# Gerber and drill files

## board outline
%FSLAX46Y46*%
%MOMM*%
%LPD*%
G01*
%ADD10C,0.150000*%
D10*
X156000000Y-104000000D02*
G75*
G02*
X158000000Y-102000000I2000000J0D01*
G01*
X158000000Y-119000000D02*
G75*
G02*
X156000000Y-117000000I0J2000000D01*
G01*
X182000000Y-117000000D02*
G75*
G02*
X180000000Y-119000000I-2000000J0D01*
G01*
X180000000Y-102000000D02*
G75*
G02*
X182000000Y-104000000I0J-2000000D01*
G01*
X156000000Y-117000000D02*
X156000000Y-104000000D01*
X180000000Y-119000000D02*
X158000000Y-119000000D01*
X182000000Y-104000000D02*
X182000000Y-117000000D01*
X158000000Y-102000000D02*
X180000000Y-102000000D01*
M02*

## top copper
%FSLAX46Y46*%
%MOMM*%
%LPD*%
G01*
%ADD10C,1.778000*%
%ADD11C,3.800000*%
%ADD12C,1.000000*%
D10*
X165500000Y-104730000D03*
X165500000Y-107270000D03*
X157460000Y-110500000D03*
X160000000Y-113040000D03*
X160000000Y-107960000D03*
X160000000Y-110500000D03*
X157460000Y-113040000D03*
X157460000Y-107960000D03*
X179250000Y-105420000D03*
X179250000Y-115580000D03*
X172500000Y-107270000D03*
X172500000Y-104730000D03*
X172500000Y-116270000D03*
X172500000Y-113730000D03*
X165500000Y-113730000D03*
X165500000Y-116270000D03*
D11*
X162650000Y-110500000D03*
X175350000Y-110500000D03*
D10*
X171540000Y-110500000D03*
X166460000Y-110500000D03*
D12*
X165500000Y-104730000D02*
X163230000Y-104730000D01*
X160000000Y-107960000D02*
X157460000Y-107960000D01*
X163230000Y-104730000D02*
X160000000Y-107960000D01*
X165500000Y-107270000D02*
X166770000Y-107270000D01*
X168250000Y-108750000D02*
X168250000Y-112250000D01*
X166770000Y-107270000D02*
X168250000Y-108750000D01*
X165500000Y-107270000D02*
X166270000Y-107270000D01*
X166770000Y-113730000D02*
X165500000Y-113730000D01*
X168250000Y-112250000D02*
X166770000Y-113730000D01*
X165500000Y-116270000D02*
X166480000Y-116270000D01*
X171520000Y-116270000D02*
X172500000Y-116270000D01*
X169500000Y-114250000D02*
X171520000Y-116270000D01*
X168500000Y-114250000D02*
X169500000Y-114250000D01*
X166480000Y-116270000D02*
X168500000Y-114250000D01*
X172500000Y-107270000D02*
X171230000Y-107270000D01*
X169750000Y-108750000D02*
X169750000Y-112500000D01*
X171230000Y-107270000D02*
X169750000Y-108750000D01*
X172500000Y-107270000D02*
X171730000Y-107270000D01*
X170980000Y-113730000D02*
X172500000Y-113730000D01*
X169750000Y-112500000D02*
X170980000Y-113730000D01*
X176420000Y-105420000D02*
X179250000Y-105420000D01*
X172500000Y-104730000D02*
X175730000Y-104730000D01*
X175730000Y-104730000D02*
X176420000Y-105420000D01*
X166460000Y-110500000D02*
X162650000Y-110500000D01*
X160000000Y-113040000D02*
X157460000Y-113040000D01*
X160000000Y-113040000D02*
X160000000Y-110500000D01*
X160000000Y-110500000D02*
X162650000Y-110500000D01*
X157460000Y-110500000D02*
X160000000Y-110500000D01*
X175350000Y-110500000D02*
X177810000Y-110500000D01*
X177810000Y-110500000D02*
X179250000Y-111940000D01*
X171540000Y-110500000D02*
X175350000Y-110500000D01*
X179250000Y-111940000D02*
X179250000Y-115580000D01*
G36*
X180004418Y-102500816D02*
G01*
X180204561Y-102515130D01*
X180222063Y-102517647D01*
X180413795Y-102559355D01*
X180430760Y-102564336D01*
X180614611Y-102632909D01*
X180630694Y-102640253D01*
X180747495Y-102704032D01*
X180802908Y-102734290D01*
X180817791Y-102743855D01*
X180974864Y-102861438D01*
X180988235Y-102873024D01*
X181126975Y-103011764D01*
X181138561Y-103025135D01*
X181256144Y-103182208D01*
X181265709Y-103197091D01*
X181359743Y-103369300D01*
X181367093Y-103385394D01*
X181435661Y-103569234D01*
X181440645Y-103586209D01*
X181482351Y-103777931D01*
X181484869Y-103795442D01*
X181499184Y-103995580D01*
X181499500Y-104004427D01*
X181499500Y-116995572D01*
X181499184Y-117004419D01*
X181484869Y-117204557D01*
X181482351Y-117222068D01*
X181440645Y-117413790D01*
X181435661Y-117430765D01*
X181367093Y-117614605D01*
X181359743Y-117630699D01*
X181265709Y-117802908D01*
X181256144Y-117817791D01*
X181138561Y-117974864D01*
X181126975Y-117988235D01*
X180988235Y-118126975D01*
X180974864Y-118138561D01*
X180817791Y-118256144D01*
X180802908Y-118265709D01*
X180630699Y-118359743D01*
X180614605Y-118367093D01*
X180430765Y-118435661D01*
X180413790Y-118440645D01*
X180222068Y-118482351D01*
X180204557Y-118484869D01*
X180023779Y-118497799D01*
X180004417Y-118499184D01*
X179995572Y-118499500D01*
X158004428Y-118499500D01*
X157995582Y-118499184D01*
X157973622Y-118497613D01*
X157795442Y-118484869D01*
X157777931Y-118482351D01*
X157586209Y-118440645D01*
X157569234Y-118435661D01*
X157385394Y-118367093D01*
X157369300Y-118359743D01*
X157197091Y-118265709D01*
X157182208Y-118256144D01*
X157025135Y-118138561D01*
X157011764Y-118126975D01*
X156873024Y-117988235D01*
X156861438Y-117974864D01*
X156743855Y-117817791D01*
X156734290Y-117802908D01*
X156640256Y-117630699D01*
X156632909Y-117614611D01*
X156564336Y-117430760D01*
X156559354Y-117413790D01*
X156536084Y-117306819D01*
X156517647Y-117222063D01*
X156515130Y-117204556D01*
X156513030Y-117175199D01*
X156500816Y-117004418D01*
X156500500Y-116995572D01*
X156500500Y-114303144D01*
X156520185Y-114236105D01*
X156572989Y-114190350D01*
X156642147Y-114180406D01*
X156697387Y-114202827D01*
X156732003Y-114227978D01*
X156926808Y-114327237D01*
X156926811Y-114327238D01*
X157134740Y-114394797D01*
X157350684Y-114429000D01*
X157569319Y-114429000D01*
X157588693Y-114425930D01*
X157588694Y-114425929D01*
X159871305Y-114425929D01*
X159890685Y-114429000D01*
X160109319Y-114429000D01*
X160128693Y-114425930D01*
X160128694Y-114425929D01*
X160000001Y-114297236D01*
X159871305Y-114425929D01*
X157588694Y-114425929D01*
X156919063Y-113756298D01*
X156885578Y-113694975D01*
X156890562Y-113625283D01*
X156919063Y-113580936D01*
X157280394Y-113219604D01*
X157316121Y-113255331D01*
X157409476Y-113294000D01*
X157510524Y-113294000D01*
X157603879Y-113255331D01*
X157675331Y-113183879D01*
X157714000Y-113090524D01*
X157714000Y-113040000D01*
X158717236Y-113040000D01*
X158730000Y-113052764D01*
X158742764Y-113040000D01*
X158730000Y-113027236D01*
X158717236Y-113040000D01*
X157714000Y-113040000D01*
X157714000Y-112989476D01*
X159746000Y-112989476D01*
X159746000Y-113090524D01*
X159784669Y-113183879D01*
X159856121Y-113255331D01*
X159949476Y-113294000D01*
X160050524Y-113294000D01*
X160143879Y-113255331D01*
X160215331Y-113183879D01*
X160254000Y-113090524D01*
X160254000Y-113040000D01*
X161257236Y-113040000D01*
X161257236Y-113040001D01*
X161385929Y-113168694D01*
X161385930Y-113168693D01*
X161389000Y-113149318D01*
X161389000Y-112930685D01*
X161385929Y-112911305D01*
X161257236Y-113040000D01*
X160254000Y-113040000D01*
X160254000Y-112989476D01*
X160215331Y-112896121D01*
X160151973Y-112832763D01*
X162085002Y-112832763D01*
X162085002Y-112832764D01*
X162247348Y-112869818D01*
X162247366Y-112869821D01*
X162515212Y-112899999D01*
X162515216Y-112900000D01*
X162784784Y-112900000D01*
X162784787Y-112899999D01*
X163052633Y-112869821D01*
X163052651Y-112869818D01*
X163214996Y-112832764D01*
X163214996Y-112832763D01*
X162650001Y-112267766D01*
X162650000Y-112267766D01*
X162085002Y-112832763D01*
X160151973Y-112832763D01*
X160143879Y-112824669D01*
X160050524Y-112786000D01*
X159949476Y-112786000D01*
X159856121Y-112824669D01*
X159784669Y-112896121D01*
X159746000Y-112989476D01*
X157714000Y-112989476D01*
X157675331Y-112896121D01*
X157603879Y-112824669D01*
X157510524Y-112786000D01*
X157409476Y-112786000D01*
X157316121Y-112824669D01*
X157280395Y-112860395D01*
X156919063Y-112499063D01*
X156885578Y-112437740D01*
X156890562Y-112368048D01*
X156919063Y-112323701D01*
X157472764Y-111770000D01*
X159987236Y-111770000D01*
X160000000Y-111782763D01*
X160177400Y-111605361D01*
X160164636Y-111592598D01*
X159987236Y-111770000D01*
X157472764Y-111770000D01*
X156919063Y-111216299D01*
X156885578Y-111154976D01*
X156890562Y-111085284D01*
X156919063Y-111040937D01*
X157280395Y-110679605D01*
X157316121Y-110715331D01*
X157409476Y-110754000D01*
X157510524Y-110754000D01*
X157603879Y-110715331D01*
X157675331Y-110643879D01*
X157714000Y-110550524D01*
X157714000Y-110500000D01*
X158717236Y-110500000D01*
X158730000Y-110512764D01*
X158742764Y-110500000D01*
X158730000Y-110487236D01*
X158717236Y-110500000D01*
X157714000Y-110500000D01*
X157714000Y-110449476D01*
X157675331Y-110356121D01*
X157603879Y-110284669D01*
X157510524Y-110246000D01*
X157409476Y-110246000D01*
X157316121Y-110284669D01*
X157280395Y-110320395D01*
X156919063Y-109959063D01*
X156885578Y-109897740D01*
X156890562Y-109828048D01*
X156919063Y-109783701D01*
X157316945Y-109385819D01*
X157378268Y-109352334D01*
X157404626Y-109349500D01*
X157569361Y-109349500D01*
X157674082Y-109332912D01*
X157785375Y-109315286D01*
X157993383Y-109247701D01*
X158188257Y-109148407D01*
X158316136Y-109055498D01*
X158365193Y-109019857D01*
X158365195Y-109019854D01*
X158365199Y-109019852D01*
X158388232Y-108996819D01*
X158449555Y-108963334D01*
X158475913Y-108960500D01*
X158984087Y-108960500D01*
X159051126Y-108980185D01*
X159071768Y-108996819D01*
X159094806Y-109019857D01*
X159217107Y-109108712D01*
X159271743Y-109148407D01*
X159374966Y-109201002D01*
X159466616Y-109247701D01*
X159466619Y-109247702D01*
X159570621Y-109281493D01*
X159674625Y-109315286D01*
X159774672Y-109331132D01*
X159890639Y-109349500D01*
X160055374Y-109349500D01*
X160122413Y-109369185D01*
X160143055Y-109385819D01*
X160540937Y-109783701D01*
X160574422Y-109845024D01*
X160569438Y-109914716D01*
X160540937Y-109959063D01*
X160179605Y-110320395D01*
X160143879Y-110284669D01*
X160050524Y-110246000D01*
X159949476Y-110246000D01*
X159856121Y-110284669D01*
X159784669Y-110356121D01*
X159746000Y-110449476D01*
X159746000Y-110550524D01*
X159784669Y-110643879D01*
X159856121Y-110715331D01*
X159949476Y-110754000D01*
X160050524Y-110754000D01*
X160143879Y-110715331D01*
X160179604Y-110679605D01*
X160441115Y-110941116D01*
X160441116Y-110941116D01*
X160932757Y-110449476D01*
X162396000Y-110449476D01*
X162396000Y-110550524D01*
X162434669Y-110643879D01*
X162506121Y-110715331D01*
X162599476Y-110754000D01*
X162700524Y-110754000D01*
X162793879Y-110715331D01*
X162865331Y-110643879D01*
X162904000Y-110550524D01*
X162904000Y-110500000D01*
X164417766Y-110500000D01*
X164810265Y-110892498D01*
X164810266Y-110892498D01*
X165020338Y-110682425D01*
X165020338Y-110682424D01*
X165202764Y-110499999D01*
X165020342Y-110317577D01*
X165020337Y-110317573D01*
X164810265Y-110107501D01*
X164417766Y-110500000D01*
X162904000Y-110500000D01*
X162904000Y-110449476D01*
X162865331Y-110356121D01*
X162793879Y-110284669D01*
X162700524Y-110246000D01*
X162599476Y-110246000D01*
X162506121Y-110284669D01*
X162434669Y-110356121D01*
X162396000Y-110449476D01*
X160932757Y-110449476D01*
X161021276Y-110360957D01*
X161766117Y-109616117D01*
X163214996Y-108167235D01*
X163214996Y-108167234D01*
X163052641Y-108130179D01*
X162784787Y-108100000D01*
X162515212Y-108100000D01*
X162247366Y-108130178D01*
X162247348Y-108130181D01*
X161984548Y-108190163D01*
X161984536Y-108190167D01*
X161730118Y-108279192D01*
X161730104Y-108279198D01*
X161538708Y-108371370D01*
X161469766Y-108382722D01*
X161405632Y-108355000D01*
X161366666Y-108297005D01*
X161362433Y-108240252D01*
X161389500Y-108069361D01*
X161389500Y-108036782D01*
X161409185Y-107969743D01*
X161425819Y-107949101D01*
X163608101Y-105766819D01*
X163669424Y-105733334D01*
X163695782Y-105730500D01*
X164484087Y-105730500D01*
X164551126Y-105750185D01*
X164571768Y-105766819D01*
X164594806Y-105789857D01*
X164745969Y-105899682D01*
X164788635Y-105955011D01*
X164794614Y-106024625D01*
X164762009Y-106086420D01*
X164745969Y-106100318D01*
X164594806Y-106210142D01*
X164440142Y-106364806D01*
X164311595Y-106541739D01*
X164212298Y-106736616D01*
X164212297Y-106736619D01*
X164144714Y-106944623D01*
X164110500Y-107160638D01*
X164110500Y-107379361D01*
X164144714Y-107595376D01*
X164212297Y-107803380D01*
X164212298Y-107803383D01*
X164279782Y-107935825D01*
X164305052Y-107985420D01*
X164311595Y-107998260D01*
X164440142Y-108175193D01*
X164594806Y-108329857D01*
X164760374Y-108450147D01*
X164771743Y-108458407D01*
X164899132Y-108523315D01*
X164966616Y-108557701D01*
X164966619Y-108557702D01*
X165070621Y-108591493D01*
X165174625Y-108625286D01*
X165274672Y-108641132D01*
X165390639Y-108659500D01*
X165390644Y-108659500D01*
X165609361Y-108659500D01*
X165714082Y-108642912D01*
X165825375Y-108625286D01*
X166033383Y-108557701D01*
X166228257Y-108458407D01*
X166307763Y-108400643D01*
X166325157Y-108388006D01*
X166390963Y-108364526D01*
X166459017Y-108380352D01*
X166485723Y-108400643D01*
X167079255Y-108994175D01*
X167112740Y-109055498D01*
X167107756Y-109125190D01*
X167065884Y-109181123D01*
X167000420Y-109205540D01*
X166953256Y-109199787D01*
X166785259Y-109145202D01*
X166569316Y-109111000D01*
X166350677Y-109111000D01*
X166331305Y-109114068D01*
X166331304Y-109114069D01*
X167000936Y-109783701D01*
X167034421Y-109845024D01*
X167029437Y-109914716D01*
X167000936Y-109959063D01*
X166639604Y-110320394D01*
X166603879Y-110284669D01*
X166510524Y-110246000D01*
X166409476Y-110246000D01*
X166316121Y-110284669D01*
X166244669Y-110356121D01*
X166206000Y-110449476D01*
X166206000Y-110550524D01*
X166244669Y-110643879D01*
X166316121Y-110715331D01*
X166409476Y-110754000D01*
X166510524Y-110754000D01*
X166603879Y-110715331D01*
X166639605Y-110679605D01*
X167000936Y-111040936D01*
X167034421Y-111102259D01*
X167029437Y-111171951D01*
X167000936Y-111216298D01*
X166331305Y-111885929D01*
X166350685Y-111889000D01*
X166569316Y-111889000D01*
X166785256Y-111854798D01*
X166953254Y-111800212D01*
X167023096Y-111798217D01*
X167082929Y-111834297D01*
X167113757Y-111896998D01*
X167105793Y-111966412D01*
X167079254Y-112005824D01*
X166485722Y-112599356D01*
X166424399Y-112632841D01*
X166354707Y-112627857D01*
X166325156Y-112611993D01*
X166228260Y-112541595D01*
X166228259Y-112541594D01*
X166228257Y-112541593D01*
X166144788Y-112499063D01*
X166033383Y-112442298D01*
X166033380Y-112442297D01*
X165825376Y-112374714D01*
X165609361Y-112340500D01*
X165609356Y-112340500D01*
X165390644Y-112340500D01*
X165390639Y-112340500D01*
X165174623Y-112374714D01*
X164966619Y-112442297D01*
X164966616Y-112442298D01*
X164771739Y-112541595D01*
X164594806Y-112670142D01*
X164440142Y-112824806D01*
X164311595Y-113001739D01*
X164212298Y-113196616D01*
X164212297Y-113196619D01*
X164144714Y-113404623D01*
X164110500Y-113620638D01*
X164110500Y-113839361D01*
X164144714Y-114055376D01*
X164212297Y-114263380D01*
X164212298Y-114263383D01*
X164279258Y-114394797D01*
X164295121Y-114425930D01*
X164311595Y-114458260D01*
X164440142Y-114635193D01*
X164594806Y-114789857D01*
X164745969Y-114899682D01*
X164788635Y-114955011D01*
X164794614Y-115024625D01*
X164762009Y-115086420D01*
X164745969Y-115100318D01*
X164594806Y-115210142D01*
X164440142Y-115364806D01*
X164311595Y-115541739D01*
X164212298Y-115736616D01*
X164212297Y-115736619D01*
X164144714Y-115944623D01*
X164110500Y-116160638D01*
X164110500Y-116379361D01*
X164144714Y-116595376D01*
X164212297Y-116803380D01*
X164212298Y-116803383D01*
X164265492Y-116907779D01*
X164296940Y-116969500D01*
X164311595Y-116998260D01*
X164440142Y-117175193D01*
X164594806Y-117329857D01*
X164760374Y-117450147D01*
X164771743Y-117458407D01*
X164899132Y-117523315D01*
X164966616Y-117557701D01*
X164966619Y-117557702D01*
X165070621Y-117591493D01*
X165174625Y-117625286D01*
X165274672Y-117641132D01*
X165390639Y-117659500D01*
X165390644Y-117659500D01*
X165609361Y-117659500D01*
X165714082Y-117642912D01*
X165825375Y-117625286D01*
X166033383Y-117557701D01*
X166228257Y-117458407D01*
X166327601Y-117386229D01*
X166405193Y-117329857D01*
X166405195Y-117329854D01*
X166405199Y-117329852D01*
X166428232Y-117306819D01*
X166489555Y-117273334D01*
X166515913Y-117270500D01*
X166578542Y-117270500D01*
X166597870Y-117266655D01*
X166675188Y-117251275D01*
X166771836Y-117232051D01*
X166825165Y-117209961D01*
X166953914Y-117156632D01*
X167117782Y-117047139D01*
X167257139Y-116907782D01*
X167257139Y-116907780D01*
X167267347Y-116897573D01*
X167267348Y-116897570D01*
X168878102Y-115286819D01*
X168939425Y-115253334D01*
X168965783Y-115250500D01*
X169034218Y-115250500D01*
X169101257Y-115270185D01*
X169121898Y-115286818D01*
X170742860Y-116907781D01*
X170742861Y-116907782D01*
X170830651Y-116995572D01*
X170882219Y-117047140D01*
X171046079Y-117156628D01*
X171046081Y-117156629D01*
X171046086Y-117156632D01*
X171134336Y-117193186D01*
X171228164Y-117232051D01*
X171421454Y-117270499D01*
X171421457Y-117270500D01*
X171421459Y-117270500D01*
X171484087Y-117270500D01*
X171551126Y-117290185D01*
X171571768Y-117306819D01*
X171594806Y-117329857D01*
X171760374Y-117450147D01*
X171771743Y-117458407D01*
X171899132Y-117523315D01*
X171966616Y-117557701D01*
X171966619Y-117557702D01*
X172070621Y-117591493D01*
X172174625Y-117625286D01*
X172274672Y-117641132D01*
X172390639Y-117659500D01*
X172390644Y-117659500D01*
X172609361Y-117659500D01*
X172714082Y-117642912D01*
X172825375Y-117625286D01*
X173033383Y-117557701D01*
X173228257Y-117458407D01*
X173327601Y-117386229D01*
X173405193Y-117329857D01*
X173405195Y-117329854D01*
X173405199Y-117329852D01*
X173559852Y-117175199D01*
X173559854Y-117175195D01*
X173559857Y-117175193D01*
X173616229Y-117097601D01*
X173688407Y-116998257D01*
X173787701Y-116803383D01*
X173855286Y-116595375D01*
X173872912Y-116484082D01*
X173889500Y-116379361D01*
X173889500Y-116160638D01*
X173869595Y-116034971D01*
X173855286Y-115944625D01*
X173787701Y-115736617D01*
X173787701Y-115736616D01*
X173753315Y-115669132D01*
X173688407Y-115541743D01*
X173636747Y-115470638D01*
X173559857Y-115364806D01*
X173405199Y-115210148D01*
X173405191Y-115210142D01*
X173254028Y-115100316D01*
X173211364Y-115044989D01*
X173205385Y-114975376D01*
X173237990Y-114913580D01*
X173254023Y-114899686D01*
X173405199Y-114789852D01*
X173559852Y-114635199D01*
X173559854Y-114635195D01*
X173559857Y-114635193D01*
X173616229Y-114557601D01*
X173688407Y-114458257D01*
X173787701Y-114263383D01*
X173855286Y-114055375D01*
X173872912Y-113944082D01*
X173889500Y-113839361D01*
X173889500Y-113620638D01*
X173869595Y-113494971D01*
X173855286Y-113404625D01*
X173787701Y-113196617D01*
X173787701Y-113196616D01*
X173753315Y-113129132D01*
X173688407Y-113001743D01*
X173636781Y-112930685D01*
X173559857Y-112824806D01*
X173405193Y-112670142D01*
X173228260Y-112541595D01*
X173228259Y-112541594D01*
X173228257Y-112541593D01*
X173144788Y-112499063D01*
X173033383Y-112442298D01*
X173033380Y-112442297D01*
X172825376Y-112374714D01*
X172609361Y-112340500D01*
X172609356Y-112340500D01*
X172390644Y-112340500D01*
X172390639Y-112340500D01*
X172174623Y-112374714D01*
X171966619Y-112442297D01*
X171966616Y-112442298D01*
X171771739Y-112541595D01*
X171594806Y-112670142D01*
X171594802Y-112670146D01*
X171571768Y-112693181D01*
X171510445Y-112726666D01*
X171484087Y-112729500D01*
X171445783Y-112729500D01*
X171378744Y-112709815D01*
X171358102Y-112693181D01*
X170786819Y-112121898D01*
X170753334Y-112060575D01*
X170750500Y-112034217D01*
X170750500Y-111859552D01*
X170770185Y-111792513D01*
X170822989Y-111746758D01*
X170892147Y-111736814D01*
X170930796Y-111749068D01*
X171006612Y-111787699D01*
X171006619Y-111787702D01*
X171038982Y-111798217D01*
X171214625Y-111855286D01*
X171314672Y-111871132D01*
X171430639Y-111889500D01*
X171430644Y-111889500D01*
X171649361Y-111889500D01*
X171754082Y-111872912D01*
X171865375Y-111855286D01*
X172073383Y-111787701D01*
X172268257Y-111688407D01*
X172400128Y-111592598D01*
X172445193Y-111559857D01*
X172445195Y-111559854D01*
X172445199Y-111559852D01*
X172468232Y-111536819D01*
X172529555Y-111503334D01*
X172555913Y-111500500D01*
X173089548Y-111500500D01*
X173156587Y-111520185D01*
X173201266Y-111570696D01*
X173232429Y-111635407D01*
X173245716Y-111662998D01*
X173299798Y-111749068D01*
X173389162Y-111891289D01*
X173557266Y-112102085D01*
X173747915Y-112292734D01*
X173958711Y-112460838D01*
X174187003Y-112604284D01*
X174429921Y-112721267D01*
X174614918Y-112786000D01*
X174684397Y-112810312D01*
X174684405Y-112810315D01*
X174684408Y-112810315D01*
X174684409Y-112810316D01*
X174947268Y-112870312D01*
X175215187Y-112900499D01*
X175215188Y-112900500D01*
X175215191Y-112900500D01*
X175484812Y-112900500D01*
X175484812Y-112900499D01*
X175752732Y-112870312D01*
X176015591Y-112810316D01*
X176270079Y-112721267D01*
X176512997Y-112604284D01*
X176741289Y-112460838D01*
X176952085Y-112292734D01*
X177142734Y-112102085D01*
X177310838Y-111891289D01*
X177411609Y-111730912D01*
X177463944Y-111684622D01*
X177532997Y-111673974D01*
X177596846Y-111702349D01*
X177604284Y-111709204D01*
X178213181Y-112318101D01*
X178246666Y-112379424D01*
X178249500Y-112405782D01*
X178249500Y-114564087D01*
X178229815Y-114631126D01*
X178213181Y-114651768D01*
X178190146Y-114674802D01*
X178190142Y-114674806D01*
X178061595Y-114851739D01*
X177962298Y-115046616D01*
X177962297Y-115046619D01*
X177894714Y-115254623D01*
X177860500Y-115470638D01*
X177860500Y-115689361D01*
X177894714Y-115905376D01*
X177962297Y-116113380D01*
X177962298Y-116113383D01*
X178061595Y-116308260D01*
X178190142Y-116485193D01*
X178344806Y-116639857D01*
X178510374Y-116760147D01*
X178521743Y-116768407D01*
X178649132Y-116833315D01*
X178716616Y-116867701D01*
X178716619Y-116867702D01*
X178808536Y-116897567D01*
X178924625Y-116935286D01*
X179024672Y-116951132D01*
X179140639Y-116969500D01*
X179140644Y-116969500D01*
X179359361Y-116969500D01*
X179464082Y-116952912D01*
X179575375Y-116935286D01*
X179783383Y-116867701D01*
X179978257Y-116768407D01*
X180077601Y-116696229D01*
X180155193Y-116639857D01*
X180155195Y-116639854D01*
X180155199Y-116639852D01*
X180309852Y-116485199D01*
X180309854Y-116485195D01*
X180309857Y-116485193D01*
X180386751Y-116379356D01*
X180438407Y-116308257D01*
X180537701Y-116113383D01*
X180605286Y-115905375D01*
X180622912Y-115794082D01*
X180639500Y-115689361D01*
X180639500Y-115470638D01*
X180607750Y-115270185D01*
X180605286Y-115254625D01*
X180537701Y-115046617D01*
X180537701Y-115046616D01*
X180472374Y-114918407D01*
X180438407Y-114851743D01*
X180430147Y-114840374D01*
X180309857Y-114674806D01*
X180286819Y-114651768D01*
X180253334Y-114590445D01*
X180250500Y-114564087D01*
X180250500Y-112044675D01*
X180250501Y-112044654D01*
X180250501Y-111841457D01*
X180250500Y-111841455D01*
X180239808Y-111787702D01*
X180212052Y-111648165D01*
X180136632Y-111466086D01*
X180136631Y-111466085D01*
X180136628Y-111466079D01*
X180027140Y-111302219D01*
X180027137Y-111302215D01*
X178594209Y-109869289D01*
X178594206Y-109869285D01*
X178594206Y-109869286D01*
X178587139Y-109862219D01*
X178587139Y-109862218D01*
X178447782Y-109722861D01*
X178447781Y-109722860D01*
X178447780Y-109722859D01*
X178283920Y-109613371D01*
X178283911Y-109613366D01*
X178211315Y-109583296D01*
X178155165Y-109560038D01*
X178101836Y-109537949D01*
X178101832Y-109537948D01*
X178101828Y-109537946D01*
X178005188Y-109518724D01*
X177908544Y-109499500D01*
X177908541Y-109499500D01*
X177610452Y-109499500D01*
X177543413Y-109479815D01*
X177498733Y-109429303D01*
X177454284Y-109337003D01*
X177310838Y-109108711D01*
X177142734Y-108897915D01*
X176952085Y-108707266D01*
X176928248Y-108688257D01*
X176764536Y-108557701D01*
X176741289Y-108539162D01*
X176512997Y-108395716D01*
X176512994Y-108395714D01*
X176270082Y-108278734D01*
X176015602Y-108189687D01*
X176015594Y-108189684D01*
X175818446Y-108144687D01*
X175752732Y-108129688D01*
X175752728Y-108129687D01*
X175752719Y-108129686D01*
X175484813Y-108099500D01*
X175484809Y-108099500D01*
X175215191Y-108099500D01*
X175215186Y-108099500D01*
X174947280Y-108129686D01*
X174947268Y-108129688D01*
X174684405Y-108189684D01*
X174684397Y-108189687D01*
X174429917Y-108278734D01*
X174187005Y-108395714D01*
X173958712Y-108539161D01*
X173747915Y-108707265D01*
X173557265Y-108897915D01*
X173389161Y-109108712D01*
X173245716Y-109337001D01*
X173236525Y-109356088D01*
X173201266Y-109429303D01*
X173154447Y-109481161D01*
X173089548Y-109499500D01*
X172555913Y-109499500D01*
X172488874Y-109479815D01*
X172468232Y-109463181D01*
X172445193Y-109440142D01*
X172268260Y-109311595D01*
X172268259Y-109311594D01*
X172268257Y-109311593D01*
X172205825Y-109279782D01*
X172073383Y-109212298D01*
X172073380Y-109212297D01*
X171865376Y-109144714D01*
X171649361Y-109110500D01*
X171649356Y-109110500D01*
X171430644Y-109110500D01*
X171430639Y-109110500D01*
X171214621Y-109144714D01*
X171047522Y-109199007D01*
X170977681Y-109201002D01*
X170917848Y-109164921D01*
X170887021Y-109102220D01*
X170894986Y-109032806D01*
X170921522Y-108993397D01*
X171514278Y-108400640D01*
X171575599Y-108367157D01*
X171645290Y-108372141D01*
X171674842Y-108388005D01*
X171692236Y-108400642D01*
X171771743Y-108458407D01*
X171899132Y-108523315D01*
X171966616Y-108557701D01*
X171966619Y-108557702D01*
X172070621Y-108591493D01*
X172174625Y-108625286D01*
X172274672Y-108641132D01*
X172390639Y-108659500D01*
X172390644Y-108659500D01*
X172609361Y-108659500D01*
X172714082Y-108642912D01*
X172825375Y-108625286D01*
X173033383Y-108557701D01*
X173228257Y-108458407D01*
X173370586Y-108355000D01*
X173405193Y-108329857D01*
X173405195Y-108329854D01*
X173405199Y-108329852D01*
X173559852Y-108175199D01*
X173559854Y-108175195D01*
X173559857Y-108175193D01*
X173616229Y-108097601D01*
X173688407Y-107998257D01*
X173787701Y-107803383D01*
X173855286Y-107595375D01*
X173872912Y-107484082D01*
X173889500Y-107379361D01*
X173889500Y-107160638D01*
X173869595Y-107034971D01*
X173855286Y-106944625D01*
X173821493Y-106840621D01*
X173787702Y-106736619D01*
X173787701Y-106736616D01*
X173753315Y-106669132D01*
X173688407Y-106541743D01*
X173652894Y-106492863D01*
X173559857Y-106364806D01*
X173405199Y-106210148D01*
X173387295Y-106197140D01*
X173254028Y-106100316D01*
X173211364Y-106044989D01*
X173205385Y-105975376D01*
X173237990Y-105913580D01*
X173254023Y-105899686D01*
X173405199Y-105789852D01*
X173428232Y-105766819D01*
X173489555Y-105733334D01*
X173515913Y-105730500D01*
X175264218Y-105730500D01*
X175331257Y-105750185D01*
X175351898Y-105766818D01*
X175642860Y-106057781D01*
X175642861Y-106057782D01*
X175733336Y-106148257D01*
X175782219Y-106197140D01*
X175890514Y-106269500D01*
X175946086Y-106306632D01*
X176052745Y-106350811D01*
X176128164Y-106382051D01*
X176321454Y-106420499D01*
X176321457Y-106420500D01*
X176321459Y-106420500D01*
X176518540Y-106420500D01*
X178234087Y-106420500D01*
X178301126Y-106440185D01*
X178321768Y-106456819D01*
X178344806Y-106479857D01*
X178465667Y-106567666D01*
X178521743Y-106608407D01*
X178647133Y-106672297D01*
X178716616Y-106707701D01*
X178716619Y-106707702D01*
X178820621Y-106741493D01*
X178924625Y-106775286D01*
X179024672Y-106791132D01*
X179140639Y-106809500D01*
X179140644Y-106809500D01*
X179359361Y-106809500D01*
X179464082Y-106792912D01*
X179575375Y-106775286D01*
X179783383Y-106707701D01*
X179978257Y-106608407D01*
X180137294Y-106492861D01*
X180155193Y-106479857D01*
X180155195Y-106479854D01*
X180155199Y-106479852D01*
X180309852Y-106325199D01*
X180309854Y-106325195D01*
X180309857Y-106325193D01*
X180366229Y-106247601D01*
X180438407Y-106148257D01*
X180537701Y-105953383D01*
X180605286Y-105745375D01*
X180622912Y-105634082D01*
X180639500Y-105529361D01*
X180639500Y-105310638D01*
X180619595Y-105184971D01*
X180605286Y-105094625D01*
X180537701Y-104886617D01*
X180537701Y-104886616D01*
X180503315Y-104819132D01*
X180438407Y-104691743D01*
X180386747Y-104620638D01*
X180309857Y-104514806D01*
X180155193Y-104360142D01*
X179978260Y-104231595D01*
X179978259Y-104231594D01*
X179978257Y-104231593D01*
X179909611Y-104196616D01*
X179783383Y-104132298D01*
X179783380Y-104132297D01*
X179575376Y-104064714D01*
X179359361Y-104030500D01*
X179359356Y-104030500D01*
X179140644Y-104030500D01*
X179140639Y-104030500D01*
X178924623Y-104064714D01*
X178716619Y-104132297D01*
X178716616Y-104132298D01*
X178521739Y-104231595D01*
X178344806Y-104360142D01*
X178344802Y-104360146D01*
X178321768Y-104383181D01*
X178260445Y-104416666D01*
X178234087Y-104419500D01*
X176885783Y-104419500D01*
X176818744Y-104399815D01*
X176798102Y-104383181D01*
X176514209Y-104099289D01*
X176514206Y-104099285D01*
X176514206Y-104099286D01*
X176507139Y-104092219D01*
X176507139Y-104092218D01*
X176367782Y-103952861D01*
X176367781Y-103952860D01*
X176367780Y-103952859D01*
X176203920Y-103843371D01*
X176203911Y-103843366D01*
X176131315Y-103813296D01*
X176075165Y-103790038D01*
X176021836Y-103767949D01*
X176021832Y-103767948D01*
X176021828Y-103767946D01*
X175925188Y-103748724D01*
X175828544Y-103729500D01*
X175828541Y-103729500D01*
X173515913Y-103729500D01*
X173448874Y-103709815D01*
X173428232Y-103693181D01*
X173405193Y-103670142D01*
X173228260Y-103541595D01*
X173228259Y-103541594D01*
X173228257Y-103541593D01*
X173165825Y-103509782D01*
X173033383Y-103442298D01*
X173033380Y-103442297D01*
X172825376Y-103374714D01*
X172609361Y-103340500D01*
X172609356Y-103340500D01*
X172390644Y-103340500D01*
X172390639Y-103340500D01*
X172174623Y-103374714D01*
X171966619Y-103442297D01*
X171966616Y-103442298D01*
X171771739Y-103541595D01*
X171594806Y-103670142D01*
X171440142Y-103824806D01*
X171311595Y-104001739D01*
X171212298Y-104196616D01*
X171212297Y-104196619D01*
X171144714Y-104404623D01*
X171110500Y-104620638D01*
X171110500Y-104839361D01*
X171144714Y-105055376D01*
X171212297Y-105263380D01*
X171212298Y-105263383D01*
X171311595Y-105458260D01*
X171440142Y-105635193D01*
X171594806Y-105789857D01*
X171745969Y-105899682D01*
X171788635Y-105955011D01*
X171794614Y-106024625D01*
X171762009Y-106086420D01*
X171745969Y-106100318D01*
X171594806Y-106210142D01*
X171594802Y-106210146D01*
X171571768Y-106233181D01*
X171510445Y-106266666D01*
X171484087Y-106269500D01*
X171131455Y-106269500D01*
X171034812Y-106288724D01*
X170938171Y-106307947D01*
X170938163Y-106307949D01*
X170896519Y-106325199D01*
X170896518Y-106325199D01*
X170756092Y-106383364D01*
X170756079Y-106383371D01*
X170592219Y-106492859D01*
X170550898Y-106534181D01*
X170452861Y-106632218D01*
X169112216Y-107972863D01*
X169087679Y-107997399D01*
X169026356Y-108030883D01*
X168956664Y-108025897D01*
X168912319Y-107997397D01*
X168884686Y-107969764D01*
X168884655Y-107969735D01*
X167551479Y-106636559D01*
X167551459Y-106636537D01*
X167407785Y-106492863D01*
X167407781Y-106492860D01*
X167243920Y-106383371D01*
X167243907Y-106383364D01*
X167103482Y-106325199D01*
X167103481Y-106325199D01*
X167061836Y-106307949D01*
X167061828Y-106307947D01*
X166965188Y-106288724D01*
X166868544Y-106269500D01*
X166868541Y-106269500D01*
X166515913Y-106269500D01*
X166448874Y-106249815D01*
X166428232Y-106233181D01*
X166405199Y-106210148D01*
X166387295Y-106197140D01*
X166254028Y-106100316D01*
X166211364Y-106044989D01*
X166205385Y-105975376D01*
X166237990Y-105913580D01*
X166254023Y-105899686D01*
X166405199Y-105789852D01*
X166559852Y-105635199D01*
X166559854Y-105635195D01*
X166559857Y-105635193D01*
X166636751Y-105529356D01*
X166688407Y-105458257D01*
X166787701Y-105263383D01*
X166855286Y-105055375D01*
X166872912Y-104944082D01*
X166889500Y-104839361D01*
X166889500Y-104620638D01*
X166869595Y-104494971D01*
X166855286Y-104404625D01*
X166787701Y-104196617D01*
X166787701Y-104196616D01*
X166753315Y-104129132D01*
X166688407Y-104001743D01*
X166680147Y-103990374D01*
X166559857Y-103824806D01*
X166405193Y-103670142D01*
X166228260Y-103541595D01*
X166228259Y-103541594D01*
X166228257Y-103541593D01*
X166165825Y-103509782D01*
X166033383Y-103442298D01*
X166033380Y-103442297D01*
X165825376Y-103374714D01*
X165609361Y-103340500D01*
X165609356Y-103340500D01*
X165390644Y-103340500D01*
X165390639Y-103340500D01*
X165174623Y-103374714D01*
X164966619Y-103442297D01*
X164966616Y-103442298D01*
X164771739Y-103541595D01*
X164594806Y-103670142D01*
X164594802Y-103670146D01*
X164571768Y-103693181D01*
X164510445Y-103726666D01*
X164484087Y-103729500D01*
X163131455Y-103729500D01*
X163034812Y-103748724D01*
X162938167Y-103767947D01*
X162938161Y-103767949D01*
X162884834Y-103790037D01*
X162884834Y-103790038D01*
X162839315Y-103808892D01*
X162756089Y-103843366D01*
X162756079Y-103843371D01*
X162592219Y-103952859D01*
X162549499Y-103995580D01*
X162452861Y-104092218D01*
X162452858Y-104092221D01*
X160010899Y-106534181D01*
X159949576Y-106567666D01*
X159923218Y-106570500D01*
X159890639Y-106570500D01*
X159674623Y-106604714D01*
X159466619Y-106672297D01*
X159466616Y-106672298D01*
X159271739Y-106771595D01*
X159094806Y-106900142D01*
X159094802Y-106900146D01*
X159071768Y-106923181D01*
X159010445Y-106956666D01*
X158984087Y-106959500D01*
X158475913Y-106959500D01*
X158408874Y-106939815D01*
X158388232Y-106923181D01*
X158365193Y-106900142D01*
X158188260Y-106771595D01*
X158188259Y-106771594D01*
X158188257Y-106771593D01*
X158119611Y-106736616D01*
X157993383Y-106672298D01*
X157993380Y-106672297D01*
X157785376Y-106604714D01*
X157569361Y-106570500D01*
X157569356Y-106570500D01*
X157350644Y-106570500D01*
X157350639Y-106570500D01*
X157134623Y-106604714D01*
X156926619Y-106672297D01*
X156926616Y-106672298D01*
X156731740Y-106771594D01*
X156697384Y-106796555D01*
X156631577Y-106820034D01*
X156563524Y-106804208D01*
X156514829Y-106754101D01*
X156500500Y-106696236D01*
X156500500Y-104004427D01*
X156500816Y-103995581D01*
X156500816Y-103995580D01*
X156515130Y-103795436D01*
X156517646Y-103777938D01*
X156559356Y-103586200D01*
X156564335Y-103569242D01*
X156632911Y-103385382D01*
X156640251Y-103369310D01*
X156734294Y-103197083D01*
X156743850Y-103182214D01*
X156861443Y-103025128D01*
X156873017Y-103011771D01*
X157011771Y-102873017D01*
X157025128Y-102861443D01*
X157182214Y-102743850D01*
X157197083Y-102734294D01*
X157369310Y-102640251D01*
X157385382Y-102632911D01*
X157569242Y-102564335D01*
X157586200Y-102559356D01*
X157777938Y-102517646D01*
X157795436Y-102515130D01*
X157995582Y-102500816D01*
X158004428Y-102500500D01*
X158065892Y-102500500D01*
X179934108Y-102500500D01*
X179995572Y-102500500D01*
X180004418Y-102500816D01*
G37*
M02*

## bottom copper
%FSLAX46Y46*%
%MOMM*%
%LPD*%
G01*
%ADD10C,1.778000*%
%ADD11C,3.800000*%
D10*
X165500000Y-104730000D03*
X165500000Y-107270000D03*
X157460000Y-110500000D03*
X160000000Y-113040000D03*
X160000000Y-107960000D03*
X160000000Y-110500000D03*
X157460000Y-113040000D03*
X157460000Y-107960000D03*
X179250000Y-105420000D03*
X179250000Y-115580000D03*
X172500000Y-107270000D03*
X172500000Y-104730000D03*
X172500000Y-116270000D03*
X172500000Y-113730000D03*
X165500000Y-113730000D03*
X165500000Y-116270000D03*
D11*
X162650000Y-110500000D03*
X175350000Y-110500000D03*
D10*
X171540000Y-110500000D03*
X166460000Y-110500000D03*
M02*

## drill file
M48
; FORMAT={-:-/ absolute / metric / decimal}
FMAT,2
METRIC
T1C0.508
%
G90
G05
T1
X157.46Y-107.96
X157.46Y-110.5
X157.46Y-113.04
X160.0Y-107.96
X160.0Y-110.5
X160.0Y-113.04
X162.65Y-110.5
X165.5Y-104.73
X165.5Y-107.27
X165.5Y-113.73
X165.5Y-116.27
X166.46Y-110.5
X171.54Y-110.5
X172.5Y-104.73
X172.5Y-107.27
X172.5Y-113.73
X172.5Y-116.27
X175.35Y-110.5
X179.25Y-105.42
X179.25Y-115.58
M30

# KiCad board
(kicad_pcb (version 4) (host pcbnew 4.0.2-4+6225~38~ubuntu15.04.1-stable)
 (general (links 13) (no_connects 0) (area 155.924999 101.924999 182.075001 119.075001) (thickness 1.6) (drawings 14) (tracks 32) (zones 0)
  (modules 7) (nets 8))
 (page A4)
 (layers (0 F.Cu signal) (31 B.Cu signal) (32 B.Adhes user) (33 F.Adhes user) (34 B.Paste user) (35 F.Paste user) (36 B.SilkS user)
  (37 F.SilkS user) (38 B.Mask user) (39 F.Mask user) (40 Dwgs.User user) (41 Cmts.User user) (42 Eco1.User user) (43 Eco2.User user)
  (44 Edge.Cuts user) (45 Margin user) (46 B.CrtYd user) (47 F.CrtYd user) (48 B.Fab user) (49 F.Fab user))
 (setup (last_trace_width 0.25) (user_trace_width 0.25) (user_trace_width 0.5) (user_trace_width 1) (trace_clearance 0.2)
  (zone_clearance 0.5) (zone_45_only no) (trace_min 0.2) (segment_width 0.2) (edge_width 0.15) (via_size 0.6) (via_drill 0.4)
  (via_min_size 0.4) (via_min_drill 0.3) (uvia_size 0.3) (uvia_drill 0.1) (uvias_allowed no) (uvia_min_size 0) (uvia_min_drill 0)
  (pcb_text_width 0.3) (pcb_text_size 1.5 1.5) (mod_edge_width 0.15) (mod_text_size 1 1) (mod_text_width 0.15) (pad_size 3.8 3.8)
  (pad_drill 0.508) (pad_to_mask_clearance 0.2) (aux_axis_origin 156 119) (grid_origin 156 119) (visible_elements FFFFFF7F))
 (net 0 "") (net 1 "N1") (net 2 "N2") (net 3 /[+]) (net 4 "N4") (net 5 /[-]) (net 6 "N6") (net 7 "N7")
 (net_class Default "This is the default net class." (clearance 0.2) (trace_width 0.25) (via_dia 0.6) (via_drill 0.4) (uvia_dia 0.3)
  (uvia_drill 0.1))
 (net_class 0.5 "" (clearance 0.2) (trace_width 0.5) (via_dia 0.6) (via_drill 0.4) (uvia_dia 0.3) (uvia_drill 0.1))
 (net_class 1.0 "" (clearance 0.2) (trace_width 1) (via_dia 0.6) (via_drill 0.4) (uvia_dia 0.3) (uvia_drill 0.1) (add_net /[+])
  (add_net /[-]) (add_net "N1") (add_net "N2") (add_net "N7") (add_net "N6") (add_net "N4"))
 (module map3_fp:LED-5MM (layer F.Cu) (at 165.5 106 270)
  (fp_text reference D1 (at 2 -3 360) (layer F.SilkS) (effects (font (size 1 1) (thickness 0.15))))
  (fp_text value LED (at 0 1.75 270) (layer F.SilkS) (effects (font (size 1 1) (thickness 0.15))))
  (pad 1 thru_hole circle (at -1.27 0 270) (size 1.778 1.778) (drill 0.508) (layers *.Cu *.Mask F.SilkS) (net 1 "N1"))
  (pad 2 thru_hole circle (at 1.27 0 270) (size 1.778 1.778) (drill 0.508) (layers *.Cu *.Mask F.SilkS) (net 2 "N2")))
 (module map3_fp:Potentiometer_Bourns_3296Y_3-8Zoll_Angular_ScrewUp (layer B.Cu) (at 160 110.5)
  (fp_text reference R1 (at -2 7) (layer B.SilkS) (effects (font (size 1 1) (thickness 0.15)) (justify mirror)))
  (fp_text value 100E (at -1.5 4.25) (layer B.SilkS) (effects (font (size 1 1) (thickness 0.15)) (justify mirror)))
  (pad 3 thru_hole circle (at -2.54 0) (size 1.778 1.778) (drill 0.508) (layers *.Cu *.Mask F.SilkS) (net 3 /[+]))
  (pad 2 thru_hole circle (at 0 2.54) (size 1.778 1.778) (drill 0.508) (layers *.Cu *.Mask F.SilkS) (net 3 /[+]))
  (pad 1 thru_hole circle (at 0 -2.54) (size 1.778 1.778) (drill 0.508) (layers *.Cu *.Mask F.SilkS) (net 1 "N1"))
  (pad 3 thru_hole circle (at 0 0) (size 1.778 1.778) (drill 0.508) (layers *.Cu *.Mask F.SilkS) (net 3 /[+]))
  (pad 2 thru_hole circle (at -2.54 2.54) (size 1.778 1.778) (drill 0.508) (layers *.Cu *.Mask B.SilkS) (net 3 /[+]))
  (pad 1 thru_hole circle (at -2.54 -2.54) (size 1.778 1.778) (drill 0.508) (layers *.Cu *.Mask B.SilkS) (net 1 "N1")))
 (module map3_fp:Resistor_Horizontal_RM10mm (layer B.Cu) (at 179.25 110.5 270)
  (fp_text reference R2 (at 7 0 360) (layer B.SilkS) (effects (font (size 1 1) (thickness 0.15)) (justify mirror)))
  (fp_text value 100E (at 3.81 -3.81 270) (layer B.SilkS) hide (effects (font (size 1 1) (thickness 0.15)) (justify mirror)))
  (pad 1 thru_hole circle (at -5.08 0 270) (size 1.778 1.778) (drill 0.508) (layers *.Cu *.Mask F.SilkS) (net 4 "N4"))
  (pad 2 thru_hole circle (at 5.08 0 270) (size 1.778 1.778) (drill 0.508) (layers *.Cu *.Mask F.SilkS) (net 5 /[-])))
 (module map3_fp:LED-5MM (layer F.Cu) (at 172.5 106 90)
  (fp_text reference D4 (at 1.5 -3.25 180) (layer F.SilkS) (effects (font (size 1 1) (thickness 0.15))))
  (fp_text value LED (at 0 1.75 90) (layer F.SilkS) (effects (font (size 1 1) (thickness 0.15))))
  (pad 1 thru_hole circle (at -1.27 0 90) (size 1.778 1.778) (drill 0.508) (layers *.Cu *.Mask F.SilkS) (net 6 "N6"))
  (pad 2 thru_hole circle (at 1.27 0 90) (size 1.778 1.778) (drill 0.508) (layers *.Cu *.Mask F.SilkS) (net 4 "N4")))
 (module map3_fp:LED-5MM (layer F.Cu) (at 172.5 115 90)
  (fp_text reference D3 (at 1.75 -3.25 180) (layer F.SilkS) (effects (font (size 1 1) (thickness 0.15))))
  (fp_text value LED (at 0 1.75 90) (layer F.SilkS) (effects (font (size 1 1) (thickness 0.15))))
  (pad 1 thru_hole circle (at -1.27 0 90) (size 1.778 1.778) (drill 0.508) (layers *.Cu *.Mask F.SilkS) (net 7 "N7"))
  (pad 2 thru_hole circle (at 1.27 0 90) (size 1.778 1.778) (drill 0.508) (layers *.Cu *.Mask F.SilkS) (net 6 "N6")))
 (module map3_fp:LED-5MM (layer F.Cu) (at 165.5 115 270)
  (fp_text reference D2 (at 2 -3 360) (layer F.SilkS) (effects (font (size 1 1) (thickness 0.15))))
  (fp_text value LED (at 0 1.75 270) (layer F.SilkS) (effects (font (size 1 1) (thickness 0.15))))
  (pad 1 thru_hole circle (at -1.27 0 270) (size 1.778 1.778) (drill 0.508) (layers *.Cu *.Mask F.SilkS) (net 2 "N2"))
  (pad 2 thru_hole circle (at 1.27 0 270) (size 1.778 1.778) (drill 0.508) (layers *.Cu *.Mask F.SilkS) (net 7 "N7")))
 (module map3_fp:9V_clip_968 (layer B.Cu) (at 169 110.5 180)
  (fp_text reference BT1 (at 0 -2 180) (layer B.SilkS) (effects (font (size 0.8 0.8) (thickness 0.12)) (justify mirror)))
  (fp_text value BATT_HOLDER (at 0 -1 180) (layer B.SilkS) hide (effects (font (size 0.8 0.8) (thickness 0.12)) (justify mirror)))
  (pad 1 thru_hole circle (at 6.35 0 180) (size 3.8 3.8) (drill 0.508) (layers *.Cu *.Mask B.SilkS) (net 3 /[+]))
  (pad 2 thru_hole circle (at -6.35 0 180) (size 3.8 3.8) (drill 0.508) (layers *.Cu *.Mask B.SilkS) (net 5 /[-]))
  (pad 2 thru_hole circle (at -2.54 0 180) (size 1.778 1.778) (drill 0.508) (layers *.Cu *.Mask F.SilkS) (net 5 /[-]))
  (pad 1 thru_hole circle (at 2.54 0 180) (size 1.778 1.778) (drill 0.508) (layers *.Cu *.Mask F.SilkS) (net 3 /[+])))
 (gr_arc (start 158 104) (end 156 104) (angle 90) (layer Edge.Cuts) (width 0.15))
 (gr_arc (start 158 117) (end 158 119) (angle 90) (layer Edge.Cuts) (width 0.15))
 (gr_arc (start 180 117) (end 182 117) (angle 90) (layer Edge.Cuts) (width 0.15))
 (gr_arc (start 180 104) (end 180 102) (angle 90) (layer Edge.Cuts) (width 0.15))
 (gr_line (start 156 117) (end 156 104) (angle 90) (layer Edge.Cuts) (width 0.15))
 (gr_line (start 180 119) (end 158 119) (angle 90) (layer Edge.Cuts) (width 0.15))
 (gr_line (start 182 104) (end 182 117) (angle 90) (layer Edge.Cuts) (width 0.15))
 (gr_line (start 158 102) (end 180 102) (angle 90) (layer Edge.Cuts) (width 0.15))
 (segment (start 165.5 104.73) (end 163.23 104.73) (width 1) (layer F.Cu) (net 1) (status 10))
 (segment (start 160 107.96) (end 157.46 107.96) (width 1) (layer F.Cu) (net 1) (status 30))
 (segment (start 163.23 104.73) (end 160 107.96) (width 1) (layer F.Cu) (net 1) (status 20))
 (segment (start 165.5 107.27) (end 166.77 107.27) (width 1) (layer F.Cu) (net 2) (status 10))
 (segment (start 168.25 108.75) (end 168.25 112.25) (width 1) (layer F.Cu) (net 2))
 (segment (start 166.77 107.27) (end 168.25 108.75) (width 1) (layer F.Cu) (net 2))
 (segment (start 165.5 107.27) (end 166.27 107.27) (width 1) (layer F.Cu) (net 2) (status 30))
 (segment (start 166.77 113.73) (end 165.5 113.73) (width 1) (layer F.Cu) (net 2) (status 20))
 (segment (start 168.25 112.25) (end 166.77 113.73) (width 1) (layer F.Cu) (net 2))
 (segment (start 165.5 116.27) (end 166.48 116.27) (width 1) (layer F.Cu) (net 7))
 (segment (start 171.52 116.27) (end 172.5 116.27) (width 1) (layer F.Cu) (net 7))
 (segment (start 169.5 114.25) (end 171.52 116.27) (width 1) (layer F.Cu) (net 7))
 (segment (start 168.5 114.25) (end 169.5 114.25) (width 1) (layer F.Cu) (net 7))
 (segment (start 166.48 116.27) (end 168.5 114.25) (width 1) (layer F.Cu) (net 7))
 (segment (start 172.5 107.27) (end 171.23 107.27) (width 1) (layer F.Cu) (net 6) (status 10))
 (segment (start 169.75 108.75) (end 169.75 112.5) (width 1) (layer F.Cu) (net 6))
 (segment (start 171.23 107.27) (end 169.75 108.75) (width 1) (layer F.Cu) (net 6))
 (segment (start 172.5 107.27) (end 171.73 107.27) (width 1) (layer F.Cu) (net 6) (status 30))
 (segment (start 170.98 113.73) (end 172.5 113.73) (width 1) (layer F.Cu) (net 6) (status 20))
 (segment (start 169.75 112.5) (end 170.98 113.73) (width 1) (layer F.Cu) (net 6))
 (segment (start 176.42 105.42) (end 179.25 105.42) (width 1) (layer F.Cu) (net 4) (status 20))
 (segment (start 172.5 104.73) (end 175.73 104.73) (width 1) (layer F.Cu) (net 4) (status 10))
 (segment (start 175.73 104.73) (end 176.42 105.42) (width 1) (layer F.Cu) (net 4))
 (segment (start 166.46 110.5) (end 162.65 110.5) (width 1) (layer F.Cu) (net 3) (status 30))
 (segment (start 160 113.04) (end 157.46 113.04) (width 1) (layer F.Cu) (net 3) (status 30))
 (segment (start 160 113.04) (end 160 110.5) (width 1) (layer F.Cu) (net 3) (status 30))
 (segment (start 160 110.5) (end 162.65 110.5) (width 1) (layer F.Cu) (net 3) (status 30))
 (segment (start 157.46 110.5) (end 160 110.5) (width 1) (layer F.Cu) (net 3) (status 30))
 (segment (start 175.35 110.5) (end 177.81 110.5) (width 1) (layer F.Cu) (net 5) (status 10))
 (segment (start 177.81 110.5) (end 179.25 111.94) (width 1) (layer F.Cu) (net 5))
 (segment (start 171.54 110.5) (end 175.35 110.5) (width 1) (layer F.Cu) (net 5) (status 30))
 (segment (start 179.25 111.94) (end 179.25 115.58) (width 1) (layer F.Cu) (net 5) (status 20))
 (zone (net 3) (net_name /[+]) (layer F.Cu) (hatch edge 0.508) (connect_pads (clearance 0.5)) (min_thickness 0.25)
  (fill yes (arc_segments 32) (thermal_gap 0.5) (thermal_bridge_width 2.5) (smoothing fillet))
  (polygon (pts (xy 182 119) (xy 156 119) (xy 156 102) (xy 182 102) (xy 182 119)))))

